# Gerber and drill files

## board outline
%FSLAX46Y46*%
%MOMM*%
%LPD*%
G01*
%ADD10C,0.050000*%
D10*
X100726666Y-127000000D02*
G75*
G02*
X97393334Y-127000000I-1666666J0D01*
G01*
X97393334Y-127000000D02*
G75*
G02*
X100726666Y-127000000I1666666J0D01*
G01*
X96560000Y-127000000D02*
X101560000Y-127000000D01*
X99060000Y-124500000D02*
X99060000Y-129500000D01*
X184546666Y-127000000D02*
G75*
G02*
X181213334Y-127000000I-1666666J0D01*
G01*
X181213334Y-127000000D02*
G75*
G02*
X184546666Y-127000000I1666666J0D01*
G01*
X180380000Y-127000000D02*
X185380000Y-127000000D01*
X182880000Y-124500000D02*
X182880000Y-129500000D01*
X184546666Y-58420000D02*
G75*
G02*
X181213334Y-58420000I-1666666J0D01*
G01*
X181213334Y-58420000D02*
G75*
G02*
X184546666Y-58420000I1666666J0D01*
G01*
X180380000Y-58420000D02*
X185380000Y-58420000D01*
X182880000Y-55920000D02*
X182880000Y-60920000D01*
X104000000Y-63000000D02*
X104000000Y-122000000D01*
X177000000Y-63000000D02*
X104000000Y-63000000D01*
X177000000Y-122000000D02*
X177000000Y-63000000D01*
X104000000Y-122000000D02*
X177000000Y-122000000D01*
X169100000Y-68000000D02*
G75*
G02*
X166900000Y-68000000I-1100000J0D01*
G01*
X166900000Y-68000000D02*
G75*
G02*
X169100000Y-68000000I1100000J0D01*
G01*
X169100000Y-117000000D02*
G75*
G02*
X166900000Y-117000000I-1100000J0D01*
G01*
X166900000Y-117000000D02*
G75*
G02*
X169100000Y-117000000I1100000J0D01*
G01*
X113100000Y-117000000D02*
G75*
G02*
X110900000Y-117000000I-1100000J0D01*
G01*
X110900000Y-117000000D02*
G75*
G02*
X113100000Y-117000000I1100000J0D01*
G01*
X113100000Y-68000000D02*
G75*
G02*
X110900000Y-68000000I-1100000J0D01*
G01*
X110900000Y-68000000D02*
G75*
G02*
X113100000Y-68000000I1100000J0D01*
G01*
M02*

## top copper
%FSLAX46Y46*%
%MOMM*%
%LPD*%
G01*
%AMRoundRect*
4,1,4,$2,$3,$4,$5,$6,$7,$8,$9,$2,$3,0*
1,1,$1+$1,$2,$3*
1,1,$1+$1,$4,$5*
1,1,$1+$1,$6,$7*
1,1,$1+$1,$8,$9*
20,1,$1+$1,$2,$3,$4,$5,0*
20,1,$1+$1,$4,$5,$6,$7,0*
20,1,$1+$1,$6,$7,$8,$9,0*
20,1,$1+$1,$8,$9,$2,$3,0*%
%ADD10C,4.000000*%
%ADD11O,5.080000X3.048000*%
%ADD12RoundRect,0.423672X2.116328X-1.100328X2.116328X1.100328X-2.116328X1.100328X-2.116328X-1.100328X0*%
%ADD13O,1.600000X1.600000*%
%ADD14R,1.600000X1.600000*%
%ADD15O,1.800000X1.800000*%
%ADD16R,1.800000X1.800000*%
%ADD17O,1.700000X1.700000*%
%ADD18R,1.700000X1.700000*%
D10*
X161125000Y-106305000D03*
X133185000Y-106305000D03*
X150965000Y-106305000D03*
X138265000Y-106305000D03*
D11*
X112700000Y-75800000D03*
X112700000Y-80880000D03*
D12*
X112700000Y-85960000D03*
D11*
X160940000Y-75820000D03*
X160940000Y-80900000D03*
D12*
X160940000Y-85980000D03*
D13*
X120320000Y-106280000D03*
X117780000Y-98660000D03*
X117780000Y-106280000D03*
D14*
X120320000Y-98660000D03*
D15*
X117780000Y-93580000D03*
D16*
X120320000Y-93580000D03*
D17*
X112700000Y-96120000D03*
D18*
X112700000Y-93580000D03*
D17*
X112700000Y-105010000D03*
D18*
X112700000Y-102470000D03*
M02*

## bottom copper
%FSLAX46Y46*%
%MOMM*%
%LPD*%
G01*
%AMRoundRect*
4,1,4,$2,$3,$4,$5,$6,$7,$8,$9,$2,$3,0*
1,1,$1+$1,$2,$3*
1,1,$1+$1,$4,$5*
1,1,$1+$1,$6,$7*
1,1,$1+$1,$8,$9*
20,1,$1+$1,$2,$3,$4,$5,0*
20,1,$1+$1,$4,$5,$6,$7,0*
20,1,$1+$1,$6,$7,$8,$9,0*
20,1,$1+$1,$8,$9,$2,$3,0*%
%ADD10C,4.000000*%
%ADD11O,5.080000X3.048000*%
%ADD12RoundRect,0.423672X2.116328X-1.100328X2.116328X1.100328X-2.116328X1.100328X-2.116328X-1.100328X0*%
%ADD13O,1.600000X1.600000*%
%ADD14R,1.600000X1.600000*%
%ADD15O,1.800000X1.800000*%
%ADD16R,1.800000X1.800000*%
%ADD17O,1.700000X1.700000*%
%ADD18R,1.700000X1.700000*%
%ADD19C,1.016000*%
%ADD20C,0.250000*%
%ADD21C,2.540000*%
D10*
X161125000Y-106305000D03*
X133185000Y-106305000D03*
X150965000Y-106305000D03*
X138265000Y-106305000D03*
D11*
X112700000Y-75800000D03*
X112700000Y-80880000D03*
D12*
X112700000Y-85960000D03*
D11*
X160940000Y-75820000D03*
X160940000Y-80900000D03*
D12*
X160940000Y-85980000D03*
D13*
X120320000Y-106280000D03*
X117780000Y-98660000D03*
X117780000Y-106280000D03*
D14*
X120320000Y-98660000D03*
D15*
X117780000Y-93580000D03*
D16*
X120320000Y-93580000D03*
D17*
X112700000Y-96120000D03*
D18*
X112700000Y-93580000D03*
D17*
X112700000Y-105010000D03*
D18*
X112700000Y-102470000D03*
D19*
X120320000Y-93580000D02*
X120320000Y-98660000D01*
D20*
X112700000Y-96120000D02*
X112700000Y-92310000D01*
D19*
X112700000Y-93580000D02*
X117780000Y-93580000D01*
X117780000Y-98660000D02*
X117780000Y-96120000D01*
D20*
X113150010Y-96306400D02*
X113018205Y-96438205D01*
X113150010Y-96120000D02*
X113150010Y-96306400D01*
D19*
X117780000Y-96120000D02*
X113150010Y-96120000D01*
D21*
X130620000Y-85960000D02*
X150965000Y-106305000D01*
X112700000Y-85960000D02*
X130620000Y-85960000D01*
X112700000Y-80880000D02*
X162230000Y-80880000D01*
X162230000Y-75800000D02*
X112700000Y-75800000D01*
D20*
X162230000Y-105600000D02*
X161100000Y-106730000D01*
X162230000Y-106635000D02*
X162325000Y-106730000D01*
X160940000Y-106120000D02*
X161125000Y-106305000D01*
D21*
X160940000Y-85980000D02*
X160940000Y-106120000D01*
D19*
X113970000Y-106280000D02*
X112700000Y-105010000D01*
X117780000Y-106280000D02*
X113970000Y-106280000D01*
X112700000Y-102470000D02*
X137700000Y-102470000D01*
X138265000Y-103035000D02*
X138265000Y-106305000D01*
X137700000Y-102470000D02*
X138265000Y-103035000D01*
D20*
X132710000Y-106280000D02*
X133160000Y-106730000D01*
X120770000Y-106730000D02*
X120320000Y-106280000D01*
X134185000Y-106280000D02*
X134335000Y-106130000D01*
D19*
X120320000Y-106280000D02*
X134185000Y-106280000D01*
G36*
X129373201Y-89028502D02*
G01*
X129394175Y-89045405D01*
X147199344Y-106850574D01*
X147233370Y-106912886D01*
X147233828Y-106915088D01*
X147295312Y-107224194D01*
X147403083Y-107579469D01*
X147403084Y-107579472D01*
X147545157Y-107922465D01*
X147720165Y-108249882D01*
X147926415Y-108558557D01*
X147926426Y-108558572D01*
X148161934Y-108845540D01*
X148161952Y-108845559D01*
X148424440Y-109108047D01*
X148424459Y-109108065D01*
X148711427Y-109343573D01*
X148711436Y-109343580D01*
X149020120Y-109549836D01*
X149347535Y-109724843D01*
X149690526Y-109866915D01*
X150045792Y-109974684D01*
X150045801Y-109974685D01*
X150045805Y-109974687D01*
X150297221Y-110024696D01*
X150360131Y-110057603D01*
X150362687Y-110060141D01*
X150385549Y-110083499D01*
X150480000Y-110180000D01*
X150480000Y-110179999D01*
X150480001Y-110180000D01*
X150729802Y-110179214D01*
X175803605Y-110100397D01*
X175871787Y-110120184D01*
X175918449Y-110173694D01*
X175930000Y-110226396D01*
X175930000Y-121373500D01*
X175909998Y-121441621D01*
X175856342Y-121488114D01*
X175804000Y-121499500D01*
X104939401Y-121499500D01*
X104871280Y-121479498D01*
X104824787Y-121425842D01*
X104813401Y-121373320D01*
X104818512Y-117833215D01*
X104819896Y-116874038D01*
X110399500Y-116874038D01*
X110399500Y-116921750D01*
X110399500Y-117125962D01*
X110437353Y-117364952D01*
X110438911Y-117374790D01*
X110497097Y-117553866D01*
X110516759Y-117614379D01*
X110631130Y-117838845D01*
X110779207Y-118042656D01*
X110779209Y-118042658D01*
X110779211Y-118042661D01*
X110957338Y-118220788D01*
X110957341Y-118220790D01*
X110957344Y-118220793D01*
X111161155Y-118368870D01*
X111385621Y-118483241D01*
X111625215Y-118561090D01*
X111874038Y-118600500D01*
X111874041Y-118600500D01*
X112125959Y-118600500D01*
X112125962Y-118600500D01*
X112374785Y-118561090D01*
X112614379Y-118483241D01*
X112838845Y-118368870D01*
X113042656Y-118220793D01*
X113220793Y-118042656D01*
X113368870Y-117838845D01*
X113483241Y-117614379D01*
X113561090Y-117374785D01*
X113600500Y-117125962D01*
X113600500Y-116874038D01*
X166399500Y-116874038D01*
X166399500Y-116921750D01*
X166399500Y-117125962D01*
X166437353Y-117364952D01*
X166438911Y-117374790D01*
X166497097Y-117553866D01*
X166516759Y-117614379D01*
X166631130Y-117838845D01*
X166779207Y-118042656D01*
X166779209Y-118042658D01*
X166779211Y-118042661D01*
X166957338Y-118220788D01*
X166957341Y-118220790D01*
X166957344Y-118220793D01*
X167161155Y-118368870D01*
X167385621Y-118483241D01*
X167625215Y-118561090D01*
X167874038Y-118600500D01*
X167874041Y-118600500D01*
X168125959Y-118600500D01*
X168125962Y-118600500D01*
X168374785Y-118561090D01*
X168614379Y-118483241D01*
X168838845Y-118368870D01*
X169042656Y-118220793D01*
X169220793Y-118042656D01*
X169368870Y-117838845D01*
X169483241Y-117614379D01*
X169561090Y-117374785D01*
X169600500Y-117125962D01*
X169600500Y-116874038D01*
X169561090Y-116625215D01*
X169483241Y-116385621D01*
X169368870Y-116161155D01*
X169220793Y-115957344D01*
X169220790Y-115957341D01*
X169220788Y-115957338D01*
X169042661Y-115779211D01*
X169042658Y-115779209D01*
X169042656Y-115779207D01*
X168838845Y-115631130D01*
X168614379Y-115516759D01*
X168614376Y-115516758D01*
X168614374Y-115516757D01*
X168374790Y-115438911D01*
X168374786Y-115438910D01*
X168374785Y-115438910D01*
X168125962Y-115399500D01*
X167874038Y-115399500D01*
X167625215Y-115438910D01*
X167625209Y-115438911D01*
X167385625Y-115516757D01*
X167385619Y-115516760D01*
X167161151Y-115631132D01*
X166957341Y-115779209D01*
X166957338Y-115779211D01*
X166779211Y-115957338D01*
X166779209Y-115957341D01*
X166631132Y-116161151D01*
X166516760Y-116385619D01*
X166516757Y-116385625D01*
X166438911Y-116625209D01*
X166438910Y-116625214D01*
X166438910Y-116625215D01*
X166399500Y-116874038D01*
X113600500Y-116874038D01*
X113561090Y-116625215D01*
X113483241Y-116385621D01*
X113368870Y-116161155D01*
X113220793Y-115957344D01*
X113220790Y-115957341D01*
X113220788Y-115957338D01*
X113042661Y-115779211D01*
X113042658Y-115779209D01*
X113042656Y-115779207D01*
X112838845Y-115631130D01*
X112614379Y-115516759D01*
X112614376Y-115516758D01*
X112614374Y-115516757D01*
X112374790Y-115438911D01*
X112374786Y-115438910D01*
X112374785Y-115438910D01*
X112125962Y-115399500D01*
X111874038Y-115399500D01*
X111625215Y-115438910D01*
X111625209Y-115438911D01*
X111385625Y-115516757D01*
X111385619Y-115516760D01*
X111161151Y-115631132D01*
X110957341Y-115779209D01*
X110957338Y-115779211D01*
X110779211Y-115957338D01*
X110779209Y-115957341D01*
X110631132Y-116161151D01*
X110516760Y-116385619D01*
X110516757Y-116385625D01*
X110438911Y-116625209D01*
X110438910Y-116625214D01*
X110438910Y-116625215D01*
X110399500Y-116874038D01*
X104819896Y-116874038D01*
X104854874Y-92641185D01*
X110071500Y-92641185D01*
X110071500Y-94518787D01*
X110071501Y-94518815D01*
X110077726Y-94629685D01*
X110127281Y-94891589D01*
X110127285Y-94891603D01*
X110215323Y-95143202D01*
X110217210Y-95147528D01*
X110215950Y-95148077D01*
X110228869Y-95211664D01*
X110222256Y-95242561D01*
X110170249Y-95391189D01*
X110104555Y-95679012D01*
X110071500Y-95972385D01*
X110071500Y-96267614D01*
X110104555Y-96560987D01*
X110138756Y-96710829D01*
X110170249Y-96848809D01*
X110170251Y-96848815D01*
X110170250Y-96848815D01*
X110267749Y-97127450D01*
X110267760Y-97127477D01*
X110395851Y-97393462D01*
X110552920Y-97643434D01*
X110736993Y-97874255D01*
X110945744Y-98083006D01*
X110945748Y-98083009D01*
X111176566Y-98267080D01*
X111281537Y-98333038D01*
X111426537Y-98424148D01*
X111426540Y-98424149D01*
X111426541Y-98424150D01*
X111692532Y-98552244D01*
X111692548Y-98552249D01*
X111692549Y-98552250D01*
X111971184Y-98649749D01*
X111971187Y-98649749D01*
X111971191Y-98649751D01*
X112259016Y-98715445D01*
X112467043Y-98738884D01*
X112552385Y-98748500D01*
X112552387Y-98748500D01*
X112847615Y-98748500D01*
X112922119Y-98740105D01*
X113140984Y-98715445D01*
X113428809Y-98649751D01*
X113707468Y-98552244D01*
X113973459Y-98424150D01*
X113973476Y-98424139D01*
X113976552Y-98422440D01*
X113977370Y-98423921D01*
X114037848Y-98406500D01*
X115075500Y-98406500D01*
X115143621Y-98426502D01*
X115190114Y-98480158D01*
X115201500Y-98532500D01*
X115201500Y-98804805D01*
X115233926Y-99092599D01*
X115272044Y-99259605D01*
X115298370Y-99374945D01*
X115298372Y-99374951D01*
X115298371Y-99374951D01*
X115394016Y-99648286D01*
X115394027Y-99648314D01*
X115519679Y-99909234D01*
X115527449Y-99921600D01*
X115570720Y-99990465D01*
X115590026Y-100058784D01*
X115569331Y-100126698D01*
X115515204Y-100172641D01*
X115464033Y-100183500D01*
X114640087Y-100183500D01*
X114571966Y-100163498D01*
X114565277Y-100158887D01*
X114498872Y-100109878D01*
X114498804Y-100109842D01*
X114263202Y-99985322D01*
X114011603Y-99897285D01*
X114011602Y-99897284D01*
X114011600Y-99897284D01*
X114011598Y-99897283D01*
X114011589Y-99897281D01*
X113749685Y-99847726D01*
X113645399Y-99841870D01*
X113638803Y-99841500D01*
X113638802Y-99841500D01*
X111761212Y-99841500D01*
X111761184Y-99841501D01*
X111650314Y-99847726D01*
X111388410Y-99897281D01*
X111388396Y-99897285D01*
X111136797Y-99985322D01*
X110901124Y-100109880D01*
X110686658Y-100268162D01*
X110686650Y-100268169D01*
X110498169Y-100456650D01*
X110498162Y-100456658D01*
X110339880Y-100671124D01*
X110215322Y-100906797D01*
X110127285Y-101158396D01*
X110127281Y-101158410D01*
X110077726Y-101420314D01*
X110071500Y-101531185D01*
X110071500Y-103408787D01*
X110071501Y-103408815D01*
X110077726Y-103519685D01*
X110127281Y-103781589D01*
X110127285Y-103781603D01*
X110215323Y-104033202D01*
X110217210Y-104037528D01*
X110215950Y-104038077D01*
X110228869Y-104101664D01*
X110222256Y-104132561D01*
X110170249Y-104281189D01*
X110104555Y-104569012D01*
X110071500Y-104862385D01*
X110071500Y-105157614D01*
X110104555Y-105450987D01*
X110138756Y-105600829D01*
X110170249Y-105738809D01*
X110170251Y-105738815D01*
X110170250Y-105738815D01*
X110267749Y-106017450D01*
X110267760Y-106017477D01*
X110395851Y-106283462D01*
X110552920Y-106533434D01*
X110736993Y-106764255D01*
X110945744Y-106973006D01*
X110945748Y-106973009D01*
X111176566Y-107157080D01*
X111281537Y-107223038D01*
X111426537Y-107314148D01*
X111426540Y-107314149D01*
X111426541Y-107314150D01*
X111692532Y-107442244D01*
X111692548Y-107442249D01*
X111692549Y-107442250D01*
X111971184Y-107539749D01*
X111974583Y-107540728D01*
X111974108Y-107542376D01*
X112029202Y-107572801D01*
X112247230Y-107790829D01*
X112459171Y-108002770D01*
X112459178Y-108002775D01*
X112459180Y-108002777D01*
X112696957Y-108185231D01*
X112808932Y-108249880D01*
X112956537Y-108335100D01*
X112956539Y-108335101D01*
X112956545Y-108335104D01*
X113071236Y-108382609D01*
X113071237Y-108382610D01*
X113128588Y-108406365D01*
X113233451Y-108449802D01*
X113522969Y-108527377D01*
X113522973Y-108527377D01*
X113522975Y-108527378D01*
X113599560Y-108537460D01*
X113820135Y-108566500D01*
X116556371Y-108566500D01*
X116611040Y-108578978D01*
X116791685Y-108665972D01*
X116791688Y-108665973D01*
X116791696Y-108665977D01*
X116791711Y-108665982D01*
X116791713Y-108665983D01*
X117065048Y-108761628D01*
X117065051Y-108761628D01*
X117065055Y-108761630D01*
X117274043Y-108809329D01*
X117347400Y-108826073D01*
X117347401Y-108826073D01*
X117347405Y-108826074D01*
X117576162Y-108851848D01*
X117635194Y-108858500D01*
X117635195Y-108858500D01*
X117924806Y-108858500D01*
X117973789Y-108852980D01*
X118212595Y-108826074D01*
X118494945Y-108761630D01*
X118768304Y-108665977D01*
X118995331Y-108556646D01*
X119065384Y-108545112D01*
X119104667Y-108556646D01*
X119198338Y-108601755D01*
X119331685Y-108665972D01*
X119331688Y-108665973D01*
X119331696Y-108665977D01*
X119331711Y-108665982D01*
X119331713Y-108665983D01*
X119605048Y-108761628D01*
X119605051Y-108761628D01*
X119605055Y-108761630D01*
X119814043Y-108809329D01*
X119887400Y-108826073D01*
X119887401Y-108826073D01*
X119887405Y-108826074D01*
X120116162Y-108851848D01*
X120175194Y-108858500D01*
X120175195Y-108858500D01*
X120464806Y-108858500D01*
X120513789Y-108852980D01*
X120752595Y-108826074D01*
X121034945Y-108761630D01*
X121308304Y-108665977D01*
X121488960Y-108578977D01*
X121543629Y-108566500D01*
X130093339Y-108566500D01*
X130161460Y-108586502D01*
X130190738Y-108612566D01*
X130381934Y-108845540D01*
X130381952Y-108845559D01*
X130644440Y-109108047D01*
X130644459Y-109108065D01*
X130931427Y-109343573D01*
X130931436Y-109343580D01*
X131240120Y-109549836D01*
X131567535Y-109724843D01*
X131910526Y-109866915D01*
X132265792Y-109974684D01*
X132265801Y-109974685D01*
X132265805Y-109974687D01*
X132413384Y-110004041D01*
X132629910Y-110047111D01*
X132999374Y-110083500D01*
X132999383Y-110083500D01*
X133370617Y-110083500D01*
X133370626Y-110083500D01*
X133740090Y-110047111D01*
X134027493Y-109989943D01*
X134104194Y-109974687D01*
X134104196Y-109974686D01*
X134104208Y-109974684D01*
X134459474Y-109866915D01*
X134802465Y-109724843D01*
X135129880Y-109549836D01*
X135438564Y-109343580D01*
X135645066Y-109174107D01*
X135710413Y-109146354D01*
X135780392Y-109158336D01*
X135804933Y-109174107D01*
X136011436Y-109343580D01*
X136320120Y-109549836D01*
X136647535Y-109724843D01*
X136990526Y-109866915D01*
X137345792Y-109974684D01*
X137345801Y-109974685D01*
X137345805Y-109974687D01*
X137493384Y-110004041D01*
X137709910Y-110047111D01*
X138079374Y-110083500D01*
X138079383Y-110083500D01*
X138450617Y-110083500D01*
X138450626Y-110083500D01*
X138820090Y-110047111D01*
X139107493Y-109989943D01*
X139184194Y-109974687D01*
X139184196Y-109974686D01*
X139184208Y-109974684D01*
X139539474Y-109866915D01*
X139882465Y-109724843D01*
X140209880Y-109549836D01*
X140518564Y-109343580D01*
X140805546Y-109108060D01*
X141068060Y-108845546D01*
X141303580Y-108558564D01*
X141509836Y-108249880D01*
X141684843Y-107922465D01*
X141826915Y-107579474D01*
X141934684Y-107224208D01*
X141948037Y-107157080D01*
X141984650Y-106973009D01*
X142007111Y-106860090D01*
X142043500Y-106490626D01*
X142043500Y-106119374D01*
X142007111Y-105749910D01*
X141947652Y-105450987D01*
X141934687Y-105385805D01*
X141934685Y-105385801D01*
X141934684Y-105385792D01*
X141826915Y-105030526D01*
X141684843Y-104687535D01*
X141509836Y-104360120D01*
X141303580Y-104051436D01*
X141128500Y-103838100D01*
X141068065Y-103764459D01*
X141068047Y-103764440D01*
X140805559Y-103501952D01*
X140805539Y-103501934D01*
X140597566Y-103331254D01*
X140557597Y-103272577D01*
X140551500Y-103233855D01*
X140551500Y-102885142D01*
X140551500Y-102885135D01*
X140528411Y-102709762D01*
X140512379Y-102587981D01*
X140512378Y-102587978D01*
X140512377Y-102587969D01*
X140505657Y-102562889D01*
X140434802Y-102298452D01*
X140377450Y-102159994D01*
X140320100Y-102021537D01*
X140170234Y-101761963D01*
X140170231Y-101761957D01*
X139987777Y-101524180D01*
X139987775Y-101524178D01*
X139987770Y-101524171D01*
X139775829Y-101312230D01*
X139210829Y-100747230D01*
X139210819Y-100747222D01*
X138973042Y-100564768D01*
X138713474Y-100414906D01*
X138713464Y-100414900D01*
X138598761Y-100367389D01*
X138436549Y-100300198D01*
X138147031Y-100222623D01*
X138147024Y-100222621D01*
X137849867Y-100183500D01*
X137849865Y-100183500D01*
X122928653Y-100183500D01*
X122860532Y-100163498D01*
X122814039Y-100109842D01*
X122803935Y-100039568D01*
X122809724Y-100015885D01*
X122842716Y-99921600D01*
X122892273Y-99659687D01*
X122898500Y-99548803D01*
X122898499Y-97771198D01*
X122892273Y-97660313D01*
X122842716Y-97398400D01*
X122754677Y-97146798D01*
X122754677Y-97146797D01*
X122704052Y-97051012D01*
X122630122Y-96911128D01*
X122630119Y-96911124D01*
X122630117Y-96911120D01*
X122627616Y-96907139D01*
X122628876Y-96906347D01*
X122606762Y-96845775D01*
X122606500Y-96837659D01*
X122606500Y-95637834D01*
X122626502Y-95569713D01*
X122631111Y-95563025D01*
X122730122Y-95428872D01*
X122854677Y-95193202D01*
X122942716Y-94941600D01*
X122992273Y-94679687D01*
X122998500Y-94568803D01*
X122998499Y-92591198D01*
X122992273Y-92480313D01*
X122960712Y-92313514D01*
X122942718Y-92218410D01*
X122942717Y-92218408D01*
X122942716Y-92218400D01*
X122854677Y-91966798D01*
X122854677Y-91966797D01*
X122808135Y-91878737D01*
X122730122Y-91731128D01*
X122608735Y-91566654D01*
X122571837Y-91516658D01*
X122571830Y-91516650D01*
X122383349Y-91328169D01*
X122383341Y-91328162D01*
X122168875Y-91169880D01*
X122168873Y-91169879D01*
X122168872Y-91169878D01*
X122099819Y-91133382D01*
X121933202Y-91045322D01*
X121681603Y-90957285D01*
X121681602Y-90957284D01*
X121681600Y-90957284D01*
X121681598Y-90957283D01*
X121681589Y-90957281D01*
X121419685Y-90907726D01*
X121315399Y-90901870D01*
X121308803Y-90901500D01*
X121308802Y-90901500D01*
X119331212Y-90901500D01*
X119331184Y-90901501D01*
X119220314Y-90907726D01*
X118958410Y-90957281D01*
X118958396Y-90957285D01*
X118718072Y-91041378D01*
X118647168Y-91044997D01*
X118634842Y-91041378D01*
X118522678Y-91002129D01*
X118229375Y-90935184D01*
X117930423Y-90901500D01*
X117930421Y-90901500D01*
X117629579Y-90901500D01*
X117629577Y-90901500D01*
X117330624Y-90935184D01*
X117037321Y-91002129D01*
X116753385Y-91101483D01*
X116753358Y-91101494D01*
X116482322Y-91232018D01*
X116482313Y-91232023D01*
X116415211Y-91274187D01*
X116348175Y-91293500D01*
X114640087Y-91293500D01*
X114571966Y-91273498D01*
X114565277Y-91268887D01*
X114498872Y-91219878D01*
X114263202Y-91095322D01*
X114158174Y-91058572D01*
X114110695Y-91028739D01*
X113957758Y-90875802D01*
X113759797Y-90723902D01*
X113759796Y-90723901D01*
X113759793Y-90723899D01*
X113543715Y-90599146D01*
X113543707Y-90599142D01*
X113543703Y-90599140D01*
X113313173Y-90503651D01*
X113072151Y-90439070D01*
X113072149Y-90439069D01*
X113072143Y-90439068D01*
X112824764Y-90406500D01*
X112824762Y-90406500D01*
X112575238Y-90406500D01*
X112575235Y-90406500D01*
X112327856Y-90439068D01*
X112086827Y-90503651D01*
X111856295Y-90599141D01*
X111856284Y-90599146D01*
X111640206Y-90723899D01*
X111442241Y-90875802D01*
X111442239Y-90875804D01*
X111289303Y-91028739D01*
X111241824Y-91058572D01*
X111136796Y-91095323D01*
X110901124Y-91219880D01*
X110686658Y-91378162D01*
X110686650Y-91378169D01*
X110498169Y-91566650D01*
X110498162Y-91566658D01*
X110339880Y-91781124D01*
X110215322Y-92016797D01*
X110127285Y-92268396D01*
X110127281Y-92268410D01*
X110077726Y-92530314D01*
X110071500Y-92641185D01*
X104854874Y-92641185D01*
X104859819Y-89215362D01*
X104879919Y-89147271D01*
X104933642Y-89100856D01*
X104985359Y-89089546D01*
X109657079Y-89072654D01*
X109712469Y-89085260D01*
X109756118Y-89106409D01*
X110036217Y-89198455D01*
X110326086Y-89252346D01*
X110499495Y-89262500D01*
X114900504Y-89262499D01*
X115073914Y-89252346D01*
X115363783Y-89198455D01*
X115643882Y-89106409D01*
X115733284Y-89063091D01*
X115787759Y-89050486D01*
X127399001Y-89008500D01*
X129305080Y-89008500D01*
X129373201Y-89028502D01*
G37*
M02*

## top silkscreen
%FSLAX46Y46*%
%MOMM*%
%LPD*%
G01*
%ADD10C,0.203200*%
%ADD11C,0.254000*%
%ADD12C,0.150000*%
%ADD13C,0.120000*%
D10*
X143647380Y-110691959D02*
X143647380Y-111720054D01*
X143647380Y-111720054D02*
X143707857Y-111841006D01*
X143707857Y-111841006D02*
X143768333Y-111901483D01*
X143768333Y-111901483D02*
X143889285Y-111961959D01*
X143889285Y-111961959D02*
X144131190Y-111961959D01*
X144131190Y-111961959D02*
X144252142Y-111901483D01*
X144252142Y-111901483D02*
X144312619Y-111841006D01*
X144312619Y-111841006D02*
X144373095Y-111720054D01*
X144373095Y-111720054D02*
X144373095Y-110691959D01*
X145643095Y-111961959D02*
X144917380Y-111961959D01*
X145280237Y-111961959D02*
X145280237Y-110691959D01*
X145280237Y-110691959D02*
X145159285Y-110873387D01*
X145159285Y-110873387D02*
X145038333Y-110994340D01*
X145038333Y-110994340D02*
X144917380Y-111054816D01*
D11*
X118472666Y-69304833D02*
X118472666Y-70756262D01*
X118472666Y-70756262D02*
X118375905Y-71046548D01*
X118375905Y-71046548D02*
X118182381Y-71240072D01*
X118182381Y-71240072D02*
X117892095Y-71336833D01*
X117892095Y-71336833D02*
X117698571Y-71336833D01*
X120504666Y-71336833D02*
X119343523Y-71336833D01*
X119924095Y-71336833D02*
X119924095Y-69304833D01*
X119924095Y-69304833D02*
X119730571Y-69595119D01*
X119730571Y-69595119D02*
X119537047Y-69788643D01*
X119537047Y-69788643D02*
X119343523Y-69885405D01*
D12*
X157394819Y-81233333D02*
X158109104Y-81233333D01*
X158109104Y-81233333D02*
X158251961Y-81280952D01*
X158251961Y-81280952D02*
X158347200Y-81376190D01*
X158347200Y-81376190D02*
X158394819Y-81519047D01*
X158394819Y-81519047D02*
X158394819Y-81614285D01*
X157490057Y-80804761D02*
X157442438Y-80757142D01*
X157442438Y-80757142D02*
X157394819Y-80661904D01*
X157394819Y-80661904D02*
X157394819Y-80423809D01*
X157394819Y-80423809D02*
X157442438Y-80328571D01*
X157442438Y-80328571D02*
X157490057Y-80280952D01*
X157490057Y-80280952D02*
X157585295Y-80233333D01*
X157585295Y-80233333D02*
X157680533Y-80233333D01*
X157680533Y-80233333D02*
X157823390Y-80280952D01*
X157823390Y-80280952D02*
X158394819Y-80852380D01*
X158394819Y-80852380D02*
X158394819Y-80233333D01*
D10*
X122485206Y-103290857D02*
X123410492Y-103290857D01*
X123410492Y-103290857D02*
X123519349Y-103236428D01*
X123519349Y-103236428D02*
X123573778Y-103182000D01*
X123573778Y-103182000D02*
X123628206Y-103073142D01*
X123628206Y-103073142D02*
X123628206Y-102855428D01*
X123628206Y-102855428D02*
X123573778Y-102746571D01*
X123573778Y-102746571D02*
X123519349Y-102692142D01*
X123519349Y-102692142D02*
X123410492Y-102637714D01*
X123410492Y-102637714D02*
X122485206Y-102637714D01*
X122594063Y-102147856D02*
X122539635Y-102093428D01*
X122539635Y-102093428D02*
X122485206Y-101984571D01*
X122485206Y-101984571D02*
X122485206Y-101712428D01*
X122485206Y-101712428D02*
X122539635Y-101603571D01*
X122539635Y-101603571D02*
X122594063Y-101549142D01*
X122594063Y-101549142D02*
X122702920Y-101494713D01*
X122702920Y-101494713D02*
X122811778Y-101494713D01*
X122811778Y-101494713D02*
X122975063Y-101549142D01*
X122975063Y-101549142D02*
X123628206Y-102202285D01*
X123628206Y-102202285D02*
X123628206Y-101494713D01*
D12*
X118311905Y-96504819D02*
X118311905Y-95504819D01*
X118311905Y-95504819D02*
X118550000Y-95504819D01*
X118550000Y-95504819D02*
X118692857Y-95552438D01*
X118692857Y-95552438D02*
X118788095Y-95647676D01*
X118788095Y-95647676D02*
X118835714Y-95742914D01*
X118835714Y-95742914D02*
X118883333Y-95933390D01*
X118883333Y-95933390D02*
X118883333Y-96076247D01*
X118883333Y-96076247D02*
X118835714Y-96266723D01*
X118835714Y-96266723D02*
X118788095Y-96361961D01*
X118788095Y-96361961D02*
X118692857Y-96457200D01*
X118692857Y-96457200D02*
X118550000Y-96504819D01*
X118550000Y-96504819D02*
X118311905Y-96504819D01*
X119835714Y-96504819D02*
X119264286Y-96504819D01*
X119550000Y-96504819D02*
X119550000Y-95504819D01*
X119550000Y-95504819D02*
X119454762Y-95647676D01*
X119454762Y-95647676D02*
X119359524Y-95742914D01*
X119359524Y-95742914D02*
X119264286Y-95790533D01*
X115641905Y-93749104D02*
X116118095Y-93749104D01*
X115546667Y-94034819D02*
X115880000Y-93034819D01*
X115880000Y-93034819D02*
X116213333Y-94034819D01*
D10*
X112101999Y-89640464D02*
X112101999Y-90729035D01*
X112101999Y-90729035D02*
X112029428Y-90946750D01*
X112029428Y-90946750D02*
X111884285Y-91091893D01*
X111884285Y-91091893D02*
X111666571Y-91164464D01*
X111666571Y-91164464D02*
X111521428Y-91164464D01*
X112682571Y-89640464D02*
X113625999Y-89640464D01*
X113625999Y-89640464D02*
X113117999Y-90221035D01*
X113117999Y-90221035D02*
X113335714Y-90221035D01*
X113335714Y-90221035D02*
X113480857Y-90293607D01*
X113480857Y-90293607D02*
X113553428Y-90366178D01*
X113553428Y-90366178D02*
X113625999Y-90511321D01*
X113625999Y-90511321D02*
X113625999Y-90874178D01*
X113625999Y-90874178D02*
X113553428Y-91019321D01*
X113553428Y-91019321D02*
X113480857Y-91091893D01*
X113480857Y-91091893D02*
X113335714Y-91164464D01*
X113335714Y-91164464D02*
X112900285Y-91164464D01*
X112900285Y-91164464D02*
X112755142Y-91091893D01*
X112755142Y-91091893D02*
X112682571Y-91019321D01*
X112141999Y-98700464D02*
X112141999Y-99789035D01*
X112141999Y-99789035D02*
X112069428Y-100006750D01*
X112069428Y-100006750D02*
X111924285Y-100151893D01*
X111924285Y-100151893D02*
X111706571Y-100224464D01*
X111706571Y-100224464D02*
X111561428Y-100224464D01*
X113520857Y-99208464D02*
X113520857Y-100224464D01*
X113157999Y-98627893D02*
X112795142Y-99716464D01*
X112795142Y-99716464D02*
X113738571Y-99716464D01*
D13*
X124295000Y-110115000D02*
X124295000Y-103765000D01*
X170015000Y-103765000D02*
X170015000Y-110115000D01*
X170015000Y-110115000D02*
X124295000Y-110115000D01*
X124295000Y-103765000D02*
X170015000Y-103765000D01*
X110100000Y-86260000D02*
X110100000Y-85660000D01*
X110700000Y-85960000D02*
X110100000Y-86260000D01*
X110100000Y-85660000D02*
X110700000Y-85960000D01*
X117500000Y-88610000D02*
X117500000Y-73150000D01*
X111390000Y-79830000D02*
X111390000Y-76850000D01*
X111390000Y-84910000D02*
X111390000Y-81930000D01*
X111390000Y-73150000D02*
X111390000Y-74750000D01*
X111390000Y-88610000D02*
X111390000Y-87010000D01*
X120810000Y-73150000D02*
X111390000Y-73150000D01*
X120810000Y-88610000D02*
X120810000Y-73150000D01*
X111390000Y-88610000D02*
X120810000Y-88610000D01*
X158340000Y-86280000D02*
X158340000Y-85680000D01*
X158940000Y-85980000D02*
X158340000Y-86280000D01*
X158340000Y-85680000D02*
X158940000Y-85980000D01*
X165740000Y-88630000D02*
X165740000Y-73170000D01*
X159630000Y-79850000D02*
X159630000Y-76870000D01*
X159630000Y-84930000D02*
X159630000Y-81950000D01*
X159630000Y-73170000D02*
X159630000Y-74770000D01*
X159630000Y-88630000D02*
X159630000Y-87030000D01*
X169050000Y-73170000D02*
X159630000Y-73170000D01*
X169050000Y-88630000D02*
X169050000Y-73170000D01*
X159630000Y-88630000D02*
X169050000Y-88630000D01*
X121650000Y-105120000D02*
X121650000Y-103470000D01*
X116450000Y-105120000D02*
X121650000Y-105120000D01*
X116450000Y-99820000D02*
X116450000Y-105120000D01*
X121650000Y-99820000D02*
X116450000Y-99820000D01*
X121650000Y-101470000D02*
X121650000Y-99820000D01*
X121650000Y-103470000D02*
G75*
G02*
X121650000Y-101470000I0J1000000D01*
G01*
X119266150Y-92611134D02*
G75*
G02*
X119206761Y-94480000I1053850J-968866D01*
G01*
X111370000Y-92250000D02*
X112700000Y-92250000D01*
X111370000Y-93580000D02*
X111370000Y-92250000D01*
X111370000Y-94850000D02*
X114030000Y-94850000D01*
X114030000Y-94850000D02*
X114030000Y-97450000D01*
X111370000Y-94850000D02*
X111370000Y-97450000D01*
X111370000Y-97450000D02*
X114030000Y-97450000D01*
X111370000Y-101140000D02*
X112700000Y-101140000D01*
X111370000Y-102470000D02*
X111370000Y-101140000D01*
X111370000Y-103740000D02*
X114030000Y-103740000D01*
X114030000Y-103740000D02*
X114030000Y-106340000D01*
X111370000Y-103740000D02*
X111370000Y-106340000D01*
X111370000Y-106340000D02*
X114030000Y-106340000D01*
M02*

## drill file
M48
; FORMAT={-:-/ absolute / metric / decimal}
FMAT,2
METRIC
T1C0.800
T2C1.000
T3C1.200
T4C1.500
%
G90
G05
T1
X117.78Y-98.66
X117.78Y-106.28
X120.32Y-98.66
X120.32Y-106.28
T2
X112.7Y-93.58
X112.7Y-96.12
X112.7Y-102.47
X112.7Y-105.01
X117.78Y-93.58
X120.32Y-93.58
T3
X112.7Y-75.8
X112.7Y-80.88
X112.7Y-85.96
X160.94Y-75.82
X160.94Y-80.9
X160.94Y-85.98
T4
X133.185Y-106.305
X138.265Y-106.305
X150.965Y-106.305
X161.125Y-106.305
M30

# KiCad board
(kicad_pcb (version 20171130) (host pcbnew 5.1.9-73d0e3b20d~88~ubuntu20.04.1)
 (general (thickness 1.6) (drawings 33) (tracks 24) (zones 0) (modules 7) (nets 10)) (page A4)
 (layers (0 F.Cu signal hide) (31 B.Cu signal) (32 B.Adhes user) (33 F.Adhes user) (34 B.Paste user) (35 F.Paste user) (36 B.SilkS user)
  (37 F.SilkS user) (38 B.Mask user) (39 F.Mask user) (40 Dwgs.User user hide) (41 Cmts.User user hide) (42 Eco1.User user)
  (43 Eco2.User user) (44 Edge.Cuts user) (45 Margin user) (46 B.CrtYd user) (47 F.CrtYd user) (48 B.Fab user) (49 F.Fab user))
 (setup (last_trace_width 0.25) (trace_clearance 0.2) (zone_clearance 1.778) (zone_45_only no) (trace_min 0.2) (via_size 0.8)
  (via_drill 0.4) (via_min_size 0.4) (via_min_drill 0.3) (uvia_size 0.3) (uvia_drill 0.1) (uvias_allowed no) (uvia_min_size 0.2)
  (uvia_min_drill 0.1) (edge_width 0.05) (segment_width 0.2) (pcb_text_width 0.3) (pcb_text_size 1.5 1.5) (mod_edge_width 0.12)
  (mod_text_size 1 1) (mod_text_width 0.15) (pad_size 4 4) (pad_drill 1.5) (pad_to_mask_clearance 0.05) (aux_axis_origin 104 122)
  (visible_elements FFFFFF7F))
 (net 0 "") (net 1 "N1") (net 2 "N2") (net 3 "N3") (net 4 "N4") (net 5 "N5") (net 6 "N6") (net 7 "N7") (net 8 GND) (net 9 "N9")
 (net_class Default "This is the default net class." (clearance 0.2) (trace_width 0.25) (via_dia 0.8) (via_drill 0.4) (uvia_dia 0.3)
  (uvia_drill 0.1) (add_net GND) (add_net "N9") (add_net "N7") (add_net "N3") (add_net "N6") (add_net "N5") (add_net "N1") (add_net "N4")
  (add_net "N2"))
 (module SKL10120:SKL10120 (layer F.Cu) (at 144.615 106.305)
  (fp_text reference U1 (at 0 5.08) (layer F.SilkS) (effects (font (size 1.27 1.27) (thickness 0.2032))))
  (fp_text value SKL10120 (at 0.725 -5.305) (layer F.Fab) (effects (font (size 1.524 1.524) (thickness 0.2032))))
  (fp_line (start -20.32 3.81) (end -20.32 -2.54) (layer F.SilkS) (width 0.12))
  (fp_line (start 25.4 -2.54) (end 25.4 3.81) (layer F.SilkS) (width 0.12))
  (fp_line (start 25.4 3.81) (end -20.32 3.81) (layer F.SilkS) (width 0.12))
  (fp_line (start -20.32 -2.54) (end 25.4 -2.54) (layer F.SilkS) (width 0.12))
  (pad 1 thru_hole circle (at 16.51 0) (size 4 4) (drill 1.5) (layers *.Cu B.Mask) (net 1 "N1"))
  (pad 4 thru_hole circle (at -11.43 0) (size 4 4) (drill 1.5) (layers *.Cu B.Mask) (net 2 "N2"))
  (pad 2 thru_hole circle (at 6.35 0) (size 4 4) (drill 1.5) (layers *.Cu B.Mask) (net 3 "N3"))
  (pad 3 thru_hole circle (at -6.35 0) (size 4 4) (drill 1.5) (layers *.Cu B.Mask) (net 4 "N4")))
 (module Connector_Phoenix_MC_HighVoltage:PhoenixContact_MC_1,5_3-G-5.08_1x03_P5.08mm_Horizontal (layer F.Cu) (at 112.7 85.96 90)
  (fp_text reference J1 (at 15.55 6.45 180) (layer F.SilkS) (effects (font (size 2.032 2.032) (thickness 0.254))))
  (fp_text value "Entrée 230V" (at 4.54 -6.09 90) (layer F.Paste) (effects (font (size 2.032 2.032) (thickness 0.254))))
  (fp_line (start -0.3 -2.6) (end 0.3 -2.6) (layer F.SilkS) (width 0.12))
  (fp_line (start 0 -2) (end -0.3 -2.6) (layer F.SilkS) (width 0.12))
  (fp_line (start 0.3 -2.6) (end 0 -2) (layer F.SilkS) (width 0.12))
  (fp_line (start -2.65 4.8) (end 12.81 4.8) (layer F.SilkS) (width 0.12))
  (fp_line (start 6.13 -1.31) (end 9.11 -1.31) (layer F.SilkS) (width 0.12))
  (fp_line (start 1.05 -1.31) (end 4.03 -1.31) (layer F.SilkS) (width 0.12))
  (fp_line (start 12.81 -1.31) (end 11.21 -1.31) (layer F.SilkS) (width 0.12))
  (fp_line (start -2.65 -1.31) (end -1.05 -1.31) (layer F.SilkS) (width 0.12))
  (fp_line (start 12.81 8.11) (end 12.81 -1.31) (layer F.SilkS) (width 0.12))
  (fp_line (start -2.65 8.11) (end 12.81 8.11) (layer F.SilkS) (width 0.12))
  (fp_line (start -2.65 -1.31) (end -2.65 8.11) (layer F.SilkS) (width 0.12))
  (pad 3 thru_hole oval (at 10.16 0 90) (size 3.048 5.08) (drill 1.2) (layers *.Cu B.Mask) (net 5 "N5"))
  (pad 2 thru_hole oval (at 5.08 0 90) (size 3.048 5.08) (drill 1.2) (layers *.Cu B.Mask) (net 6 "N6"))
  (pad 1 thru_hole roundrect (at 0 0 90) (size 3.048 5.08) (drill 1.2) (layers *.Cu B.Mask) (roundrect_rratio 0.139) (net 3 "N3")))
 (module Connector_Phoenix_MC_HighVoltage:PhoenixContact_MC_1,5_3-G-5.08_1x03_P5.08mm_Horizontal (layer F.Cu) (at 160.94 85.98 90)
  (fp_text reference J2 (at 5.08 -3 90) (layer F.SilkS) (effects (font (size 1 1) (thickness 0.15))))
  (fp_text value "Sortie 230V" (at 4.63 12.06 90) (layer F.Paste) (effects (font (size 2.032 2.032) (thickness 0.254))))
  (fp_line (start -0.3 -2.6) (end 0.3 -2.6) (layer F.SilkS) (width 0.12))
  (fp_line (start 0 -2) (end -0.3 -2.6) (layer F.SilkS) (width 0.12))
  (fp_line (start 0.3 -2.6) (end 0 -2) (layer F.SilkS) (width 0.12))
  (fp_line (start -2.65 4.8) (end 12.81 4.8) (layer F.SilkS) (width 0.12))
  (fp_line (start 6.13 -1.31) (end 9.11 -1.31) (layer F.SilkS) (width 0.12))
  (fp_line (start 1.05 -1.31) (end 4.03 -1.31) (layer F.SilkS) (width 0.12))
  (fp_line (start 12.81 -1.31) (end 11.21 -1.31) (layer F.SilkS) (width 0.12))
  (fp_line (start -2.65 -1.31) (end -1.05 -1.31) (layer F.SilkS) (width 0.12))
  (fp_line (start 12.81 8.11) (end 12.81 -1.31) (layer F.SilkS) (width 0.12))
  (fp_line (start -2.65 8.11) (end 12.81 8.11) (layer F.SilkS) (width 0.12))
  (fp_line (start -2.65 -1.31) (end -2.65 8.11) (layer F.SilkS) (width 0.12))
  (pad 3 thru_hole oval (at 10.16 0 90) (size 3.048 5.08) (drill 1.2) (layers *.Cu B.Mask) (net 5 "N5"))
  (pad 2 thru_hole oval (at 5.08 0 90) (size 3.048 5.08) (drill 1.2) (layers *.Cu B.Mask) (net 6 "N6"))
  (pad 1 thru_hole roundrect (at 0 0 90) (size 3.048 5.08) (drill 1.2) (layers *.Cu B.Mask) (roundrect_rratio 0.139) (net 1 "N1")))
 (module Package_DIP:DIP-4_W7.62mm (layer F.Cu) (at 120.32 98.66 270)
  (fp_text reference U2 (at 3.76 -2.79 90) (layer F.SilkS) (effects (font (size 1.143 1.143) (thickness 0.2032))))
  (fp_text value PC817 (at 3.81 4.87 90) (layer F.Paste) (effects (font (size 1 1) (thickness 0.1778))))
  (fp_line (start 6.46 -1.33) (end 4.81 -1.33) (layer F.SilkS) (width 0.12))
  (fp_line (start 6.46 3.87) (end 6.46 -1.33) (layer F.SilkS) (width 0.12))
  (fp_line (start 1.16 3.87) (end 6.46 3.87) (layer F.SilkS) (width 0.12))
  (fp_line (start 1.16 -1.33) (end 1.16 3.87) (layer F.SilkS) (width 0.12))
  (fp_line (start 2.81 -1.33) (end 1.16 -1.33) (layer F.SilkS) (width 0.12))
  (fp_arc (start 3.81 -1.33) (end 2.81 -1.33) (angle -180) (layer F.SilkS) (width 0.12))
  (pad 4 thru_hole oval (at 7.62 0 270) (size 1.6 1.6) (drill 0.8) (layers *.Cu B.Mask) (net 2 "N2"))
  (pad 2 thru_hole oval (at 0 2.54 270) (size 1.6 1.6) (drill 0.8) (layers *.Cu B.Mask) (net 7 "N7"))
  (pad 3 thru_hole oval (at 7.62 2.54 270) (size 1.6 1.6) (drill 0.8) (layers *.Cu B.Mask) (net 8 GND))
  (pad 1 thru_hole rect (at 0 0 270) (size 1.6 1.6) (drill 0.8) (layers *.Cu B.Mask) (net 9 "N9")))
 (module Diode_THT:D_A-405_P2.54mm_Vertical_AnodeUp (layer F.Cu) (at 120.32 93.58 180)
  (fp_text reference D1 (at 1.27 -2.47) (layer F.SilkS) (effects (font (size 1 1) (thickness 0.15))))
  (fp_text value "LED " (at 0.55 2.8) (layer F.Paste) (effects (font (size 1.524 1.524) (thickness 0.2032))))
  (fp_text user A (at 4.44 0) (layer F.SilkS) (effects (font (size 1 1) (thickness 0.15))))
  (fp_arc (start 0 0) (end 1.113239 -0.9) (angle -278.451986) (layer F.SilkS) (width 0.12))
  (pad 2 thru_hole oval (at 2.54 0 180) (size 1.8 1.8) (drill 1) (layers *.Cu B.Mask) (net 7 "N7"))
  (pad 1 thru_hole rect (at 0 0 180) (size 1.8 1.8) (drill 1) (layers *.Cu B.Mask) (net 9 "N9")))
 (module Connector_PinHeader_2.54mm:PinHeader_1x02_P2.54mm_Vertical (layer F.Cu) (at 112.7 93.58)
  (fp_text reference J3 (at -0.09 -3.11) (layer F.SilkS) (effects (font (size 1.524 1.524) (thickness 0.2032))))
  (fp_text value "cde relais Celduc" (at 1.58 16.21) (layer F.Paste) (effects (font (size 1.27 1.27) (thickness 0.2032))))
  (fp_line (start -1.33 -1.33) (end 0 -1.33) (layer F.SilkS) (width 0.12))
  (fp_line (start -1.33 0) (end -1.33 -1.33) (layer F.SilkS) (width 0.12))
  (fp_line (start -1.33 1.27) (end 1.33 1.27) (layer F.SilkS) (width 0.12))
  (fp_line (start 1.33 1.27) (end 1.33 3.87) (layer F.SilkS) (width 0.12))
  (fp_line (start -1.33 1.27) (end -1.33 3.87) (layer F.SilkS) (width 0.12))
  (fp_line (start -1.33 3.87) (end 1.33 3.87) (layer F.SilkS) (width 0.12))
  (pad 2 thru_hole oval (at 0 2.54) (size 1.7 1.7) (drill 1) (layers *.Cu B.Mask) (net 7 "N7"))
  (pad 1 thru_hole rect (at 0 0) (size 1.7 1.7) (drill 1) (layers *.Cu B.Mask) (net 7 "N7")))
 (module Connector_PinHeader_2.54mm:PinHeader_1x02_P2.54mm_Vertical (layer F.Cu) (at 112.7 102.47)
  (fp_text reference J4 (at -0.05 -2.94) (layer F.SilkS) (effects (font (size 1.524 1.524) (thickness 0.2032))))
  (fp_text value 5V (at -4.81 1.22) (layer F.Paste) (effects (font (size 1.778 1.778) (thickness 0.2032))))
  (fp_line (start -1.33 -1.33) (end 0 -1.33) (layer F.SilkS) (width 0.12))
  (fp_line (start -1.33 0) (end -1.33 -1.33) (layer F.SilkS) (width 0.12))
  (fp_line (start -1.33 1.27) (end 1.33 1.27) (layer F.SilkS) (width 0.12))
  (fp_line (start 1.33 1.27) (end 1.33 3.87) (layer F.SilkS) (width 0.12))
  (fp_line (start -1.33 1.27) (end -1.33 3.87) (layer F.SilkS) (width 0.12))
  (fp_line (start -1.33 3.87) (end 1.33 3.87) (layer F.SilkS) (width 0.12))
  (pad 2 thru_hole oval (at 0 2.54) (size 1.7 1.7) (drill 1) (layers *.Cu B.Mask) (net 8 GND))
  (pad 1 thru_hole rect (at 0 0) (size 1.7 1.7) (drill 1) (layers *.Cu B.Mask) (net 4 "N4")))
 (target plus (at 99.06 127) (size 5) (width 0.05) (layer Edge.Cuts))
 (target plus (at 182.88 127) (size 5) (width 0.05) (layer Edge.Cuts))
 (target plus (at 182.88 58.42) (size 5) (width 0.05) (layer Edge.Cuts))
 (gr_line (start 104 63) (end 104 122) (layer Edge.Cuts) (width 0.05))
 (gr_line (start 177 63) (end 104 63) (layer Edge.Cuts) (width 0.05))
 (gr_line (start 177 122) (end 177 63) (layer Edge.Cuts) (width 0.05))
 (gr_line (start 104 122) (end 177 122) (layer Edge.Cuts) (width 0.05))
 (gr_circle (center 168 68) (end 169.1 68) (layer Edge.Cuts) (width 0.05))
 (gr_circle (center 168 117) (end 169.1 117) (layer Edge.Cuts) (width 0.05))
 (gr_circle (center 112 117) (end 113.1 117) (layer Edge.Cuts) (width 0.05))
 (gr_circle (center 112 68) (end 113.1 68) (layer Edge.Cuts) (width 0.05))
 (segment (start 120.32 93.58) (end 120.32 98.66) (width 1.016) (layer B.Cu) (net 9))
 (segment (start 112.7 96.12) (end 112.7 92.31) (width 0.25) (layer B.Cu) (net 7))
 (segment (start 112.7 93.58) (end 117.78 93.58) (width 1.016) (layer B.Cu) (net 7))
 (segment (start 117.78 98.66) (end 117.78 96.12) (width 1.016) (layer B.Cu) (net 7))
 (segment (start 113.15001 96.3064) (end 113.018205 96.438205) (width 0.25) (layer B.Cu) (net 7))
 (segment (start 113.15001 96.12) (end 113.15001 96.3064) (width 0.25) (layer B.Cu) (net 7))
 (segment (start 117.78 96.12) (end 113.15001 96.12) (width 1.016) (layer B.Cu) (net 7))
 (segment (start 130.62 85.96) (end 150.965 106.305) (width 2.54) (layer B.Cu) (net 3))
 (segment (start 112.7 85.96) (end 130.62 85.96) (width 2.54) (layer B.Cu) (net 3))
 (segment (start 112.7 80.88) (end 162.23 80.88) (width 2.54) (layer B.Cu) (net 6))
 (segment (start 162.23 75.8) (end 112.7 75.8) (width 2.54) (layer B.Cu) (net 5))
 (segment (start 162.23 105.6) (end 161.1 106.73) (width 0.25) (layer B.Cu) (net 1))
 (segment (start 162.23 106.635) (end 162.325 106.73) (width 0.25) (layer B.Cu) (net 1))
 (segment (start 160.94 106.12) (end 161.125 106.305) (width 0.25) (layer B.Cu) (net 1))
 (segment (start 160.94 85.98) (end 160.94 106.12) (width 2.54) (layer B.Cu) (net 1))
 (segment (start 113.97 106.28) (end 112.7 105.01) (width 1.016) (layer B.Cu) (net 8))
 (segment (start 117.78 106.28) (end 113.97 106.28) (width 1.016) (layer B.Cu) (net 8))
 (segment (start 112.7 102.47) (end 137.7 102.47) (width 1.016) (layer B.Cu) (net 4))
 (segment (start 138.265 103.035) (end 138.265 106.305) (width 1.016) (layer B.Cu) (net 4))
 (segment (start 137.7 102.47) (end 138.265 103.035) (width 1.016) (layer B.Cu) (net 4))
 (segment (start 132.71 106.28) (end 133.16 106.73) (width 0.25) (layer B.Cu) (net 2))
 (segment (start 120.77 106.73) (end 120.32 106.28) (width 0.25) (layer B.Cu) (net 2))
 (segment (start 134.185 106.28) (end 134.335 106.13) (width 0.25) (layer B.Cu) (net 2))
 (segment (start 120.32 106.28) (end 134.185 106.28) (width 1.016) (layer B.Cu) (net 2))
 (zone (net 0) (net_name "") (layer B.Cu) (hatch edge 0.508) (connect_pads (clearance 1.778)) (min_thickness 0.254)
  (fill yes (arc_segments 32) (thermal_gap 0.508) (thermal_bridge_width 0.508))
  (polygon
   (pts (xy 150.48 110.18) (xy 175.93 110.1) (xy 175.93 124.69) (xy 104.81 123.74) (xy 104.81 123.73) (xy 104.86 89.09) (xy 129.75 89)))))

